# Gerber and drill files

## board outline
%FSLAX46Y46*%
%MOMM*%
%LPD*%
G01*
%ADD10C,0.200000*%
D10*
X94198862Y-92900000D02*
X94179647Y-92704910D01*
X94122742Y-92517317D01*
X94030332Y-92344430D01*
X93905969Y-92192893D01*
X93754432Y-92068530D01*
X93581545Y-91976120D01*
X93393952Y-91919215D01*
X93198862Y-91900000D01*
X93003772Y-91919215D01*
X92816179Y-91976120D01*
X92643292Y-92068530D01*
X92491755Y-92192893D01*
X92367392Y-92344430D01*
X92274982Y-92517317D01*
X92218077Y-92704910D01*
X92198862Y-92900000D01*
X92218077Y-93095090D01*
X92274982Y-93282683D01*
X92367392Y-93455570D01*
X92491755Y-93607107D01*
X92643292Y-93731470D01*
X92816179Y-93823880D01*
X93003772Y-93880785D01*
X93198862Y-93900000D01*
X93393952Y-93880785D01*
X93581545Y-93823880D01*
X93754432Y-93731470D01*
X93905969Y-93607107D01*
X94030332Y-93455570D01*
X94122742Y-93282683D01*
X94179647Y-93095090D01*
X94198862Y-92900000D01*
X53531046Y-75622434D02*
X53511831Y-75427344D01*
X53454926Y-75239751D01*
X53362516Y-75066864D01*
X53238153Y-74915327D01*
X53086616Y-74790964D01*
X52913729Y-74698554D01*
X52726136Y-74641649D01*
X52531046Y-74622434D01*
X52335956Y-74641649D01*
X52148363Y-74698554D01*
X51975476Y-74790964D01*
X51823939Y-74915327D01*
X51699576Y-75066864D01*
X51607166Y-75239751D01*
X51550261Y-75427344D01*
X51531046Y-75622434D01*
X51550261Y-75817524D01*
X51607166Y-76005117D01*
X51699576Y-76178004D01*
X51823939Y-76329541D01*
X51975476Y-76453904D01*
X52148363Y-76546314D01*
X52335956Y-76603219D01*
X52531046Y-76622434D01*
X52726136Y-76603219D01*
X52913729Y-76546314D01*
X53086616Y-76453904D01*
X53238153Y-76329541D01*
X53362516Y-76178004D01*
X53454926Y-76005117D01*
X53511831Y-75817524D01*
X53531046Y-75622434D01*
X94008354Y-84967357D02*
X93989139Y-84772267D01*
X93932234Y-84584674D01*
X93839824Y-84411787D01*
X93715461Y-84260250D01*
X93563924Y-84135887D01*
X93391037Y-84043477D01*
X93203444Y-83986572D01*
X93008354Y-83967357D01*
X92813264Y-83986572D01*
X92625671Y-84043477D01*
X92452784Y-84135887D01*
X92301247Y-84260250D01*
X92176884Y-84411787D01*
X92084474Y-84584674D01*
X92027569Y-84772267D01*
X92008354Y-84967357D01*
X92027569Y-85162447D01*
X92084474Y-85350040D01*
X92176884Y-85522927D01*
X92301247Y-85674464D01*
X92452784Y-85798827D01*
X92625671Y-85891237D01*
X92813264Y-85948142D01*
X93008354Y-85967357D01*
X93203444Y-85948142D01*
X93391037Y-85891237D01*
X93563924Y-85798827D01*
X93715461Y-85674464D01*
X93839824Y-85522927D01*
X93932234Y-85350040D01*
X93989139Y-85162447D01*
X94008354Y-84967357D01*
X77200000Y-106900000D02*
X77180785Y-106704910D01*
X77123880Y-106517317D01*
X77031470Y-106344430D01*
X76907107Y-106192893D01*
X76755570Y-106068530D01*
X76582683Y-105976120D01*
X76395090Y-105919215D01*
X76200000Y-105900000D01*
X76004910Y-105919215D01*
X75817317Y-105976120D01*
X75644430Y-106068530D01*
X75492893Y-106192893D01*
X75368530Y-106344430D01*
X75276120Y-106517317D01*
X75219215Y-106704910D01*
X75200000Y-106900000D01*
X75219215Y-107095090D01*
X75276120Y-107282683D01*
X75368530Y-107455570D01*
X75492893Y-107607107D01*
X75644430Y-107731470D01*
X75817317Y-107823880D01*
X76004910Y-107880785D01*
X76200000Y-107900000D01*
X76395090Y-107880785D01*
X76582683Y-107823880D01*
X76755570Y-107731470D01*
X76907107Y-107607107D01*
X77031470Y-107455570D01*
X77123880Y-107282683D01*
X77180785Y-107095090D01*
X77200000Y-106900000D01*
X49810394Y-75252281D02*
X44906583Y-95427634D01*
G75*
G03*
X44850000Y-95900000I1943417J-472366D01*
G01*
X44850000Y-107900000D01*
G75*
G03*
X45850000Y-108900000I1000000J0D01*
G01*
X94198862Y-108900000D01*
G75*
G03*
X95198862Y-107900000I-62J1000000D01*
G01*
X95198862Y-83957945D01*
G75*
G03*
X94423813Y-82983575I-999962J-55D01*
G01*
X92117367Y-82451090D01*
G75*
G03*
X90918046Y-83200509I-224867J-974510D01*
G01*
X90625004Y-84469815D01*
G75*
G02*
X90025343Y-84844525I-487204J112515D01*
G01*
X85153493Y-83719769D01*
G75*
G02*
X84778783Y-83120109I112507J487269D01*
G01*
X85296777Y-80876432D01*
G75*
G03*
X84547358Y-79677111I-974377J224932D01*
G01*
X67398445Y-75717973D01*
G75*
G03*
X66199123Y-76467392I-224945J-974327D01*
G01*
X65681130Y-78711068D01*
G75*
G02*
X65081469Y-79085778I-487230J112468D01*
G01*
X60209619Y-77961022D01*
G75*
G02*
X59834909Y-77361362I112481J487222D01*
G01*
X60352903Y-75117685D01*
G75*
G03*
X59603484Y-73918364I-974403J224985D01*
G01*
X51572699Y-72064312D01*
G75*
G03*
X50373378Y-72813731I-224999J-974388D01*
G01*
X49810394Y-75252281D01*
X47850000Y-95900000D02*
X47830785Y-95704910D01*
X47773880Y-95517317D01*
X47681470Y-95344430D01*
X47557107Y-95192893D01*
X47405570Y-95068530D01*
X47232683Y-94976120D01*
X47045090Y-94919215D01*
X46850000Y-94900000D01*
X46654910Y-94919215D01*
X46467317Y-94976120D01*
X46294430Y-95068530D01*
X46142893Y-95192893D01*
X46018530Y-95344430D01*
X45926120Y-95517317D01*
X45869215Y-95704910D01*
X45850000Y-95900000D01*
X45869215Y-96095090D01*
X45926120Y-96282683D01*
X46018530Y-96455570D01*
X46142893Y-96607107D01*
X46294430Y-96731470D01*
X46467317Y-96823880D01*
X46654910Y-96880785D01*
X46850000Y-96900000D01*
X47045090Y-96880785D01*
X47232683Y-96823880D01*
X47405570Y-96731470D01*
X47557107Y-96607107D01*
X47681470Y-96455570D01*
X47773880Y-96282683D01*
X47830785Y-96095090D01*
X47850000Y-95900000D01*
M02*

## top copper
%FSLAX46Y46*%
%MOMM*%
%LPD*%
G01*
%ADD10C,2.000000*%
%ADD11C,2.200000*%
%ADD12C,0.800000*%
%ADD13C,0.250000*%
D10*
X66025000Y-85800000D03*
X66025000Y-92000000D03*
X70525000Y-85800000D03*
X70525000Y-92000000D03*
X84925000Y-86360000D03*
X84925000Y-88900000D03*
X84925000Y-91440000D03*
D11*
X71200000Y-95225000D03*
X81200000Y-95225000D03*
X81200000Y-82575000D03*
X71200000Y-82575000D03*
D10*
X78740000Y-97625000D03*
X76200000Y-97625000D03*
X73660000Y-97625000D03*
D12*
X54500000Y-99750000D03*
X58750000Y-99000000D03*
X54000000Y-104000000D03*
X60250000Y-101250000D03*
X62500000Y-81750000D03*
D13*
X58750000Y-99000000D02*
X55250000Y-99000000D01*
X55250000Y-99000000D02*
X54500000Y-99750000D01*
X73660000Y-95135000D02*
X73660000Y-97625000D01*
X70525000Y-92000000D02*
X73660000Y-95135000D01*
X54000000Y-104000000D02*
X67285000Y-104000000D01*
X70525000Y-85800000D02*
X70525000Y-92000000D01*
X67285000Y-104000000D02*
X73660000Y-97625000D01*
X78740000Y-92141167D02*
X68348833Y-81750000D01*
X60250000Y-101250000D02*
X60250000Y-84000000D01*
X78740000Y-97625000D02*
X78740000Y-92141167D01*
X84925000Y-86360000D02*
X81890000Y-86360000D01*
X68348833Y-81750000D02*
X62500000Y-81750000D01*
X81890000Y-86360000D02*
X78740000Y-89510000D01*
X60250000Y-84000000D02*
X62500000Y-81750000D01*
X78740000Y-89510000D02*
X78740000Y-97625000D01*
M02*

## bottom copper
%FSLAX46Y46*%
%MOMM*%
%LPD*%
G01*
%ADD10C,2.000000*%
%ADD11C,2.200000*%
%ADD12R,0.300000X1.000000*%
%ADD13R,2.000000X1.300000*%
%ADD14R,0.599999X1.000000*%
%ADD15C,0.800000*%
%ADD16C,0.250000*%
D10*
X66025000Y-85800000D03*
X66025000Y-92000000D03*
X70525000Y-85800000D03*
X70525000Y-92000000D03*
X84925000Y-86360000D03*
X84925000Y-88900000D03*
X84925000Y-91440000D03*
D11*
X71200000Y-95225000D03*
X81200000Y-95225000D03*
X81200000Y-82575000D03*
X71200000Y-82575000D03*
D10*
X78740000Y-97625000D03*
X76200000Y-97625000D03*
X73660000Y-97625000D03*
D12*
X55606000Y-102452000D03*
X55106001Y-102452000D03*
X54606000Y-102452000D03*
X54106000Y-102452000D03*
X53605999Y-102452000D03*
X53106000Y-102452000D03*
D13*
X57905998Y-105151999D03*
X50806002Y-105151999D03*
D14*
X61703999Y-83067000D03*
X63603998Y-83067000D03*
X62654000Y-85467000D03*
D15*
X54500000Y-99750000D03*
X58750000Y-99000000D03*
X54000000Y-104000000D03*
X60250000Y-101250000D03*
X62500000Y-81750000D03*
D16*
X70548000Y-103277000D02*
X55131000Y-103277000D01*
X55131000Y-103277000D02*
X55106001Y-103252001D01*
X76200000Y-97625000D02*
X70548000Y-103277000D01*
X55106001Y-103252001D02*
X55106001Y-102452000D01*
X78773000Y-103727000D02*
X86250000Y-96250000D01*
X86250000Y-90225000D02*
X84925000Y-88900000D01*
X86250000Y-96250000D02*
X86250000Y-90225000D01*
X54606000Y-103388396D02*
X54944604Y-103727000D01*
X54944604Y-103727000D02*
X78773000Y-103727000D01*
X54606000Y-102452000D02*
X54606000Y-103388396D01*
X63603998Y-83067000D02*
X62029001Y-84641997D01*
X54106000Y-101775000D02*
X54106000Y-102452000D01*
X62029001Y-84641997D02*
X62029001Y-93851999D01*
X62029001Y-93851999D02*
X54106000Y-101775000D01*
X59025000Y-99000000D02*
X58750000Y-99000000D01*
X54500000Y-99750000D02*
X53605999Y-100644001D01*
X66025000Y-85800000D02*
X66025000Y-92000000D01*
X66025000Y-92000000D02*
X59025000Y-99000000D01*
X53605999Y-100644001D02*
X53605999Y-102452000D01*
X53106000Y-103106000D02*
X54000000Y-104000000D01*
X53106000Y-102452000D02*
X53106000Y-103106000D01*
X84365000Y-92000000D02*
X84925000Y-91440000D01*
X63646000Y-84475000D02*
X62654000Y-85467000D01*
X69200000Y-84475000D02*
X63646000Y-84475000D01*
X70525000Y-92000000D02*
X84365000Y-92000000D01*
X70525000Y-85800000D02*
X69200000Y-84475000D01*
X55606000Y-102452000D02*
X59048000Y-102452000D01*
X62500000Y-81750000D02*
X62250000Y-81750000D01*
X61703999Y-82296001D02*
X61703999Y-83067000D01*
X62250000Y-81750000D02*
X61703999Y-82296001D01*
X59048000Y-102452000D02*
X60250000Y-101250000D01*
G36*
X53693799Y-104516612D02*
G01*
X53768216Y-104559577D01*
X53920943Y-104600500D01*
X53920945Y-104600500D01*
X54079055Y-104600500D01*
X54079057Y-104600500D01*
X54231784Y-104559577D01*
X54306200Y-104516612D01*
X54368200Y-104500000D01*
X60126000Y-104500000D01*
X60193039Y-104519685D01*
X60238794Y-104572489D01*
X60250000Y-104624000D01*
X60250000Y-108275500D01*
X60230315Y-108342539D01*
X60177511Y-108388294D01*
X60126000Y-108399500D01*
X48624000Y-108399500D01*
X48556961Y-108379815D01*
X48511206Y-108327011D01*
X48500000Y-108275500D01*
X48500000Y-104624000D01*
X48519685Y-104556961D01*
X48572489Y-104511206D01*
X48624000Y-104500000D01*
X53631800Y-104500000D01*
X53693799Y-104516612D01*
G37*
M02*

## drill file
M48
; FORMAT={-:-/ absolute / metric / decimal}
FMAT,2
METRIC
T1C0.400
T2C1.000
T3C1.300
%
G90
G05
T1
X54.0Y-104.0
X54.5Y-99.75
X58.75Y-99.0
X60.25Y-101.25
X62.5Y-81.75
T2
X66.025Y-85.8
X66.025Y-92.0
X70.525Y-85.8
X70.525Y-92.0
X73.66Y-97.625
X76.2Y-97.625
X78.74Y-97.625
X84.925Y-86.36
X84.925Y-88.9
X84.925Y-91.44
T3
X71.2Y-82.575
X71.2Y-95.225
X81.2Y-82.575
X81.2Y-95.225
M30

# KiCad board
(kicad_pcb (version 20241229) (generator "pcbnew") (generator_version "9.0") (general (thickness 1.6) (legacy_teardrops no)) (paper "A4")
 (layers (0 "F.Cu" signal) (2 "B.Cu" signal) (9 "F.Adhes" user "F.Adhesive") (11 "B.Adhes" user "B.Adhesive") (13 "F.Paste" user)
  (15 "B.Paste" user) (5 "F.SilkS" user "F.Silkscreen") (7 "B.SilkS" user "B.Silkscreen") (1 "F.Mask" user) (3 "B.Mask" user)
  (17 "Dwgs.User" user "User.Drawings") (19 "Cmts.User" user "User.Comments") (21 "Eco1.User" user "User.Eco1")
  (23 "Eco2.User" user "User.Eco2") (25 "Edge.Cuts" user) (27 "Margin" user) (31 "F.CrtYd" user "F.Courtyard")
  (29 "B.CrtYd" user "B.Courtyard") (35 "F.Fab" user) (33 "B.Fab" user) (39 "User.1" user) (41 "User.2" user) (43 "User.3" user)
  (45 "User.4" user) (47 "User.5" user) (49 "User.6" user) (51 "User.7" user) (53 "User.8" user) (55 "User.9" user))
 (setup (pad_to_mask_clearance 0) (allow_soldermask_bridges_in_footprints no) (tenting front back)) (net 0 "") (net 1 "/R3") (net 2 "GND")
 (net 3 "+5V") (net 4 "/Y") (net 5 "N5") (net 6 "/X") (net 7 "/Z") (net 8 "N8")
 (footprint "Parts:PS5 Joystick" (layer "F.Cu") (at 76.2 88.9)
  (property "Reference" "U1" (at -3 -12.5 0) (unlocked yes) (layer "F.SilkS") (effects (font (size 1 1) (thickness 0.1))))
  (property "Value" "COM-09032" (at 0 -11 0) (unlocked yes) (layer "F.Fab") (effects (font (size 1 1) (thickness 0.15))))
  (pad "B1A" thru_hole circle (at -10.175 -3.1) (size 2 2) (drill 1) (layers "*.Cu" "*.Mask") (remove_unused_layers no) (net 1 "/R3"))
  (pad "B1A" thru_hole circle (at -10.175 3.1) (size 2 2) (drill 1) (layers "*.Cu" "*.Mask") (remove_unused_layers no) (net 1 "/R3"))
  (pad "B2A" thru_hole circle (at -5.675 -3.1) (size 2 2) (drill 1) (layers "*.Cu" "*.Mask") (remove_unused_layers no) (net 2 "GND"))
  (pad "B2A" thru_hole circle (at -5.675 3.1) (size 2 2) (drill 1) (layers "*.Cu" "*.Mask") (remove_unused_layers no) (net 2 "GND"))
  (pad "H1" thru_hole circle (at 8.725 -2.54) (size 2 2) (drill 1) (layers "*.Cu" "*.Mask") (remove_unused_layers no) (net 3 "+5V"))
  (pad "H2" thru_hole circle (at 8.725 0) (size 2 2) (drill 1) (layers "*.Cu" "*.Mask") (remove_unused_layers no) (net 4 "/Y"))
  (pad "H3" thru_hole circle (at 8.725 2.54) (size 2 2) (drill 1) (layers "*.Cu" "*.Mask") (remove_unused_layers no) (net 2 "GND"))
  (pad "S1" thru_hole circle (at -5 6.325) (size 2.2 2.2) (drill 1.3) (layers "*.Cu" "*.Mask") (remove_unused_layers no) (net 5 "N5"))
  (pad "S2" thru_hole circle (at 5 6.325) (size 2.2 2.2) (drill 1.3) (layers "*.Cu" "*.Mask") (remove_unused_layers no) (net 5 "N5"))
  (pad "S3" thru_hole circle (at 5 -6.325) (size 2.2 2.2) (drill 1.3) (layers "*.Cu" "*.Mask") (remove_unused_layers no) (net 5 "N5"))
  (pad "S4" thru_hole circle (at -5 -6.325) (size 2.2 2.2) (drill 1.3) (layers "*.Cu" "*.Mask") (remove_unused_layers no) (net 5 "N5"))
  (pad "V1" thru_hole circle (at 2.54 8.725) (size 2 2) (drill 1) (layers "*.Cu" "*.Mask") (remove_unused_layers no) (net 3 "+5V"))
  (pad "V2" thru_hole circle (at 0 8.725) (size 2 2) (drill 1) (layers "*.Cu" "*.Mask") (remove_unused_layers no) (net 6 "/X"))
  (pad "V3" thru_hole circle (at -2.54 8.725) (size 2 2) (drill 1) (layers "*.Cu" "*.Mask") (remove_unused_layers no) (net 2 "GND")))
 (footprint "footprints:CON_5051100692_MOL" (layer "B.Cu") (at 54.356 104.902 180)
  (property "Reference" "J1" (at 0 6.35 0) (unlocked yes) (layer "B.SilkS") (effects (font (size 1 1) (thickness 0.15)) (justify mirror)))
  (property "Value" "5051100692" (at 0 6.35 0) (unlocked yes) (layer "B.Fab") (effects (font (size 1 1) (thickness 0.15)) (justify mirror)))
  (pad "1" smd rect (at -1.25 2.45 180) (size 0.3 1) (layers "B.Cu" "B.Mask" "B.Paste") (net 3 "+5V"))
  (pad "2" smd rect (at -0.750001 2.45 180) (size 0.3 1) (layers "B.Cu" "B.Mask" "B.Paste") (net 6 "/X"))
  (pad "3" smd rect (at -0.25 2.45 180) (size 0.3 1) (layers "B.Cu" "B.Mask" "B.Paste") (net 4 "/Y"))
  (pad "4" smd rect (at 0.25 2.45 180) (size 0.3 1) (layers "B.Cu" "B.Mask" "B.Paste") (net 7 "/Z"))
  (pad "5" smd rect (at 0.750001 2.45 180) (size 0.3 1) (layers "B.Cu" "B.Mask" "B.Paste") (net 1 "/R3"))
  (pad "6" smd rect (at 1.25 2.45 180) (size 0.3 1) (layers "B.Cu" "B.Mask" "B.Paste") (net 2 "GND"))
  (pad "P1" smd rect (at -3.549998 -0.249999 180) (size 2 1.3) (layers "B.Cu" "B.Mask" "B.Paste") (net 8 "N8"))
  (pad "P2" smd rect (at 3.549998 -0.249999 180) (size 2 1.3) (layers "B.Cu" "B.Mask" "B.Paste") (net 8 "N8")))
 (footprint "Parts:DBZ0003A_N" (layer "B.Cu") (at 62.654 84.267 -90)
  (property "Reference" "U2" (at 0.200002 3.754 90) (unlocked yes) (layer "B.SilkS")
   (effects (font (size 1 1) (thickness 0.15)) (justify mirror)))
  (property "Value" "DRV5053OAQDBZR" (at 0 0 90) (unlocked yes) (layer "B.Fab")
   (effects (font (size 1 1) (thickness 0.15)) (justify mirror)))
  (pad "1" smd rect (at -1.2 0.950001 180) (size 0.599999 1) (layers "B.Cu" "B.Mask" "B.Paste") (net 3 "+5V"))
  (pad "2" smd rect (at -1.2 -0.949998 180) (size 0.599999 1) (layers "B.Cu" "B.Mask" "B.Paste") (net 7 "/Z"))
  (pad "3" smd rect (at 1.2 0 180) (size 0.599999 1) (layers "B.Cu" "B.Mask" "B.Paste") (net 2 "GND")))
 (gr_poly
  (pts (xy 94.198862 92.9) (xy 94.179647 92.70491) (xy 94.122742 92.517317) (xy 94.030332 92.34443) (xy 93.905969 92.192893)
   (xy 93.754432 92.06853) (xy 93.581545 91.97612) (xy 93.393952 91.919215) (xy 93.198862 91.9) (xy 93.003772 91.919215)
   (xy 92.816179 91.97612) (xy 92.643292 92.06853) (xy 92.491755 92.192893) (xy 92.367392 92.34443) (xy 92.274982 92.517317)
   (xy 92.218077 92.70491) (xy 92.198862 92.9) (xy 92.218077 93.09509) (xy 92.274982 93.282683) (xy 92.367392 93.45557)
   (xy 92.491755 93.607107) (xy 92.643292 93.73147) (xy 92.816179 93.82388) (xy 93.003772 93.880785) (xy 93.198862 93.9)
   (xy 93.393952 93.880785) (xy 93.581545 93.82388) (xy 93.754432 93.73147) (xy 93.905969 93.607107) (xy 94.030332 93.45557)
   (xy 94.122742 93.282683) (xy 94.179647 93.09509) (xy 94.198862 92.9))
  (stroke (width 0.2) (type solid)) (fill no) (layer "Edge.Cuts"))
 (gr_poly
  (pts (xy 53.531046 75.622434) (xy 53.511831 75.427344) (xy 53.454926 75.239751) (xy 53.362516 75.066864) (xy 53.238153 74.915327)
   (xy 53.086616 74.790964) (xy 52.913729 74.698554) (xy 52.726136 74.641649) (xy 52.531046 74.622434) (xy 52.335956 74.641649)
   (xy 52.148363 74.698554) (xy 51.975476 74.790964) (xy 51.823939 74.915327) (xy 51.699576 75.066864) (xy 51.607166 75.239751)
   (xy 51.550261 75.427344) (xy 51.531046 75.622434) (xy 51.550261 75.817524) (xy 51.607166 76.005117) (xy 51.699576 76.178004)
   (xy 51.823939 76.329541) (xy 51.975476 76.453904) (xy 52.148363 76.546314) (xy 52.335956 76.603219) (xy 52.531046 76.622434)
   (xy 52.726136 76.603219) (xy 52.913729 76.546314) (xy 53.086616 76.453904) (xy 53.238153 76.329541) (xy 53.362516 76.178004)
   (xy 53.454926 76.005117) (xy 53.511831 75.817524) (xy 53.531046 75.622434))
  (stroke (width 0.2) (type solid)) (fill no) (layer "Edge.Cuts"))
 (gr_poly
  (pts (xy 94.008354 84.967357) (xy 93.989139 84.772267) (xy 93.932234 84.584674) (xy 93.839824 84.411787) (xy 93.715461 84.26025)
   (xy 93.563924 84.135887) (xy 93.391037 84.043477) (xy 93.203444 83.986572) (xy 93.008354 83.967357) (xy 92.813264 83.986572)
   (xy 92.625671 84.043477) (xy 92.452784 84.135887) (xy 92.301247 84.26025) (xy 92.176884 84.411787) (xy 92.084474 84.584674)
   (xy 92.027569 84.772267) (xy 92.008354 84.967357) (xy 92.027569 85.162447) (xy 92.084474 85.35004) (xy 92.176884 85.522927)
   (xy 92.301247 85.674464) (xy 92.452784 85.798827) (xy 92.625671 85.891237) (xy 92.813264 85.948142) (xy 93.008354 85.967357)
   (xy 93.203444 85.948142) (xy 93.391037 85.891237) (xy 93.563924 85.798827) (xy 93.715461 85.674464) (xy 93.839824 85.522927)
   (xy 93.932234 85.35004) (xy 93.989139 85.162447) (xy 94.008354 84.967357))
  (stroke (width 0.2) (type solid)) (fill no) (layer "Edge.Cuts"))
 (gr_poly
  (pts (xy 77.2 106.9) (xy 77.180785 106.70491) (xy 77.12388 106.517317) (xy 77.03147 106.34443) (xy 76.907107 106.192893)
   (xy 76.75557 106.06853) (xy 76.582683 105.97612) (xy 76.39509 105.919215) (xy 76.2 105.9) (xy 76.00491 105.919215)
   (xy 75.817317 105.97612) (xy 75.64443 106.06853) (xy 75.492893 106.192893) (xy 75.36853 106.34443) (xy 75.27612 106.517317)
   (xy 75.219215 106.70491) (xy 75.2 106.9) (xy 75.219215 107.09509) (xy 75.27612 107.282683) (xy 75.36853 107.45557)
   (xy 75.492893 107.607107) (xy 75.64443 107.73147) (xy 75.817317 107.82388) (xy 76.00491 107.880785) (xy 76.2 107.9)
   (xy 76.39509 107.880785) (xy 76.582683 107.82388) (xy 76.75557 107.73147) (xy 76.907107 107.607107) (xy 77.03147 107.45557)
   (xy 77.12388 107.282683) (xy 77.180785 107.09509) (xy 77.2 106.9))
  (stroke (width 0.2) (type solid)) (fill no) (layer "Edge.Cuts"))
 (gr_poly
  (pts (xy 49.810394 75.252281)
   (arc (start 44.906583 95.427634) (mid 44.864196 95.662129) (end 44.85 95.9))
   (arc (start 44.85 107.9) (mid 45.142893 108.607107) (end 45.85 108.9))
   (arc (start 94.198862 108.9) (mid 94.905966 108.607093) (end 95.198862 107.9))
   (arc (start 95.198862 83.957945) (mid 94.981467 83.335431) (end 94.423813 82.983575))
   (arc (start 92.117367 82.45109) (mid 91.362505 82.577445) (end 90.918046 83.200509))
   (arc (start 90.625004 84.469815) (mid 90.402771 84.781349) (end 90.025343 84.844525))
   (arc (start 85.153493 83.719769) (mid 84.841972 83.497537) (end 84.778783 83.120109))
   (arc (start 85.296777 80.876432) (mid 85.170456 80.121561) (end 84.547358 79.677111))
   (arc (start 67.398445 75.717973) (mid 66.643574 75.844295) (end 66.199123 76.467392))
   (arc (start 65.68113 78.711068) (mid 65.458904 79.022617) (end 65.081469 79.085778))
   (arc (start 60.209619 77.961022) (mid 59.89807 77.738797) (end 59.834909 77.361362))
   (arc (start 60.352903 75.117685) (mid 60.226581 74.362815) (end 59.603484 73.918364))
   (arc (start 51.572699 72.064312) (mid 50.817829 72.190634) (end 50.373378 72.813731)))
  (stroke (width 0.2) (type solid)) (fill no) (layer "Edge.Cuts"))
 (gr_poly
  (pts (xy 47.85 95.9) (xy 47.830785 95.70491) (xy 47.77388 95.517317) (xy 47.68147 95.34443) (xy 47.557107 95.192893)
   (xy 47.40557 95.06853) (xy 47.232683 94.97612) (xy 47.04509 94.919215) (xy 46.85 94.9) (xy 46.65491 94.919215) (xy 46.467317 94.97612)
   (xy 46.29443 95.06853) (xy 46.142893 95.192893) (xy 46.01853 95.34443) (xy 45.92612 95.517317) (xy 45.869215 95.70491) (xy 45.85 95.9)
   (xy 45.869215 96.09509) (xy 45.92612 96.282683) (xy 46.01853 96.45557) (xy 46.142893 96.607107) (xy 46.29443 96.73147)
   (xy 46.467317 96.82388) (xy 46.65491 96.880785) (xy 46.85 96.9) (xy 47.04509 96.880785) (xy 47.232683 96.82388) (xy 47.40557 96.73147)
   (xy 47.557107 96.607107) (xy 47.68147 96.45557) (xy 47.77388 96.282683) (xy 47.830785 96.09509) (xy 47.85 95.9))
  (stroke (width 0.2) (type solid)) (fill no) (layer "Edge.Cuts"))
 (segment (start 70.548 103.277) (end 55.131 103.277) (width 0.25) (layer "B.Cu") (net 6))
 (segment (start 55.131 103.277) (end 55.106001 103.252001) (width 0.25) (layer "B.Cu") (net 6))
 (segment (start 76.2 97.625) (end 70.548 103.277) (width 0.25) (layer "B.Cu") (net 6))
 (segment (start 55.106001 103.252001) (end 55.106001 102.452) (width 0.25) (layer "B.Cu") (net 6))
 (segment (start 78.773 103.727) (end 86.25 96.25) (width 0.25) (layer "B.Cu") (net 4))
 (segment (start 86.25 90.225) (end 84.925 88.9) (width 0.25) (layer "B.Cu") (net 4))
 (segment (start 86.25 96.25) (end 86.25 90.225) (width 0.25) (layer "B.Cu") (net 4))
 (segment (start 54.606 103.388396) (end 54.944604 103.727) (width 0.25) (layer "B.Cu") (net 4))
 (segment (start 54.944604 103.727) (end 78.773 103.727) (width 0.25) (layer "B.Cu") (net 4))
 (segment (start 54.606 102.452) (end 54.606 103.388396) (width 0.25) (layer "B.Cu") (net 4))
 (segment (start 63.603998 83.067) (end 62.029001 84.641997) (width 0.25) (layer "B.Cu") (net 7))
 (segment (start 54.106 101.775) (end 54.106 102.452) (width 0.25) (layer "B.Cu") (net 7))
 (segment (start 62.029001 84.641997) (end 62.029001 93.851999) (width 0.25) (layer "B.Cu") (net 7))
 (segment (start 62.029001 93.851999) (end 54.106 101.775) (width 0.25) (layer "B.Cu") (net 7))
 (segment (start 58.75 99) (end 55.25 99) (width 0.25) (layer "F.Cu") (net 1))
 (segment (start 55.25 99) (end 54.5 99.75) (width 0.25) (layer "F.Cu") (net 1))
 (via (at 54.5 99.75) (size 0.8) (drill 0.4) (layers "F.Cu" "B.Cu") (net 1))
 (via (at 58.75 99) (size 0.8) (drill 0.4) (layers "F.Cu" "B.Cu") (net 1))
 (segment (start 59.025 99) (end 58.75 99) (width 0.25) (layer "B.Cu") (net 1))
 (segment (start 54.5 99.75) (end 53.605999 100.644001) (width 0.25) (layer "B.Cu") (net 1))
 (segment (start 66.025 85.8) (end 66.025 92) (width 0.25) (layer "B.Cu") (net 1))
 (segment (start 66.025 92) (end 59.025 99) (width 0.25) (layer "B.Cu") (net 1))
 (segment (start 53.605999 100.644001) (end 53.605999 102.452) (width 0.25) (layer "B.Cu") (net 1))
 (segment (start 73.66 95.135) (end 73.66 97.625) (width 0.25) (layer "F.Cu") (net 2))
 (segment (start 70.525 92) (end 73.66 95.135) (width 0.25) (layer "F.Cu") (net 2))
 (segment (start 54 104) (end 67.285 104) (width 0.25) (layer "F.Cu") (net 2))
 (segment (start 70.525 85.8) (end 70.525 92) (width 0.25) (layer "F.Cu") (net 2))
 (segment (start 67.285 104) (end 73.66 97.625) (width 0.25) (layer "F.Cu") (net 2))
 (via (at 54 104) (size 0.8) (drill 0.4) (layers "F.Cu" "B.Cu") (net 2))
 (segment (start 53.106 103.106) (end 54 104) (width 0.25) (layer "B.Cu") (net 2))
 (segment (start 53.106 102.452) (end 53.106 103.106) (width 0.25) (layer "B.Cu") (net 2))
 (segment (start 84.365 92) (end 84.925 91.44) (width 0.25) (layer "B.Cu") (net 2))
 (segment (start 63.646 84.475) (end 62.654 85.467) (width 0.25) (layer "B.Cu") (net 2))
 (segment (start 69.2 84.475) (end 63.646 84.475) (width 0.25) (layer "B.Cu") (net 2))
 (segment (start 70.525 92) (end 84.365 92) (width 0.25) (layer "B.Cu") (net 2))
 (segment (start 70.525 85.8) (end 69.2 84.475) (width 0.25) (layer "B.Cu") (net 2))
 (segment (start 78.74 92.141167) (end 68.348833 81.75) (width 0.25) (layer "F.Cu") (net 3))
 (segment (start 60.25 101.25) (end 60.25 84) (width 0.25) (layer "F.Cu") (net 3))
 (segment (start 78.74 97.625) (end 78.74 92.141167) (width 0.25) (layer "F.Cu") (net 3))
 (segment (start 84.925 86.36) (end 81.89 86.36) (width 0.25) (layer "F.Cu") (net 3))
 (segment (start 68.348833 81.75) (end 62.5 81.75) (width 0.25) (layer "F.Cu") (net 3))
 (segment (start 81.89 86.36) (end 78.74 89.51) (width 0.25) (layer "F.Cu") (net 3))
 (segment (start 60.25 84) (end 62.5 81.75) (width 0.25) (layer "F.Cu") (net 3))
 (segment (start 78.74 89.51) (end 78.74 97.625) (width 0.25) (layer "F.Cu") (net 3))
 (via (at 60.25 101.25) (size 0.8) (drill 0.4) (layers "F.Cu" "B.Cu") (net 3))
 (via (at 62.5 81.75) (size 0.8) (drill 0.4) (layers "F.Cu" "B.Cu") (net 3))
 (segment (start 55.606 102.452) (end 59.048 102.452) (width 0.25) (layer "B.Cu") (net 3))
 (segment (start 62.5 81.75) (end 62.25 81.75) (width 0.25) (layer "B.Cu") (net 3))
 (segment (start 61.703999 82.296001) (end 61.703999 83.067) (width 0.25) (layer "B.Cu") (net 3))
 (segment (start 62.25 81.75) (end 61.703999 82.296001) (width 0.25) (layer "B.Cu") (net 3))
 (segment (start 59.048 102.452) (end 60.25 101.25) (width 0.25) (layer "B.Cu") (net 3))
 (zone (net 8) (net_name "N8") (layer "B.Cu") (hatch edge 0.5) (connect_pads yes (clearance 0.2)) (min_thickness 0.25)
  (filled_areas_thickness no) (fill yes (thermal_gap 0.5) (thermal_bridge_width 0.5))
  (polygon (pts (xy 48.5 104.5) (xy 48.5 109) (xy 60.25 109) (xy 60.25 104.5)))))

